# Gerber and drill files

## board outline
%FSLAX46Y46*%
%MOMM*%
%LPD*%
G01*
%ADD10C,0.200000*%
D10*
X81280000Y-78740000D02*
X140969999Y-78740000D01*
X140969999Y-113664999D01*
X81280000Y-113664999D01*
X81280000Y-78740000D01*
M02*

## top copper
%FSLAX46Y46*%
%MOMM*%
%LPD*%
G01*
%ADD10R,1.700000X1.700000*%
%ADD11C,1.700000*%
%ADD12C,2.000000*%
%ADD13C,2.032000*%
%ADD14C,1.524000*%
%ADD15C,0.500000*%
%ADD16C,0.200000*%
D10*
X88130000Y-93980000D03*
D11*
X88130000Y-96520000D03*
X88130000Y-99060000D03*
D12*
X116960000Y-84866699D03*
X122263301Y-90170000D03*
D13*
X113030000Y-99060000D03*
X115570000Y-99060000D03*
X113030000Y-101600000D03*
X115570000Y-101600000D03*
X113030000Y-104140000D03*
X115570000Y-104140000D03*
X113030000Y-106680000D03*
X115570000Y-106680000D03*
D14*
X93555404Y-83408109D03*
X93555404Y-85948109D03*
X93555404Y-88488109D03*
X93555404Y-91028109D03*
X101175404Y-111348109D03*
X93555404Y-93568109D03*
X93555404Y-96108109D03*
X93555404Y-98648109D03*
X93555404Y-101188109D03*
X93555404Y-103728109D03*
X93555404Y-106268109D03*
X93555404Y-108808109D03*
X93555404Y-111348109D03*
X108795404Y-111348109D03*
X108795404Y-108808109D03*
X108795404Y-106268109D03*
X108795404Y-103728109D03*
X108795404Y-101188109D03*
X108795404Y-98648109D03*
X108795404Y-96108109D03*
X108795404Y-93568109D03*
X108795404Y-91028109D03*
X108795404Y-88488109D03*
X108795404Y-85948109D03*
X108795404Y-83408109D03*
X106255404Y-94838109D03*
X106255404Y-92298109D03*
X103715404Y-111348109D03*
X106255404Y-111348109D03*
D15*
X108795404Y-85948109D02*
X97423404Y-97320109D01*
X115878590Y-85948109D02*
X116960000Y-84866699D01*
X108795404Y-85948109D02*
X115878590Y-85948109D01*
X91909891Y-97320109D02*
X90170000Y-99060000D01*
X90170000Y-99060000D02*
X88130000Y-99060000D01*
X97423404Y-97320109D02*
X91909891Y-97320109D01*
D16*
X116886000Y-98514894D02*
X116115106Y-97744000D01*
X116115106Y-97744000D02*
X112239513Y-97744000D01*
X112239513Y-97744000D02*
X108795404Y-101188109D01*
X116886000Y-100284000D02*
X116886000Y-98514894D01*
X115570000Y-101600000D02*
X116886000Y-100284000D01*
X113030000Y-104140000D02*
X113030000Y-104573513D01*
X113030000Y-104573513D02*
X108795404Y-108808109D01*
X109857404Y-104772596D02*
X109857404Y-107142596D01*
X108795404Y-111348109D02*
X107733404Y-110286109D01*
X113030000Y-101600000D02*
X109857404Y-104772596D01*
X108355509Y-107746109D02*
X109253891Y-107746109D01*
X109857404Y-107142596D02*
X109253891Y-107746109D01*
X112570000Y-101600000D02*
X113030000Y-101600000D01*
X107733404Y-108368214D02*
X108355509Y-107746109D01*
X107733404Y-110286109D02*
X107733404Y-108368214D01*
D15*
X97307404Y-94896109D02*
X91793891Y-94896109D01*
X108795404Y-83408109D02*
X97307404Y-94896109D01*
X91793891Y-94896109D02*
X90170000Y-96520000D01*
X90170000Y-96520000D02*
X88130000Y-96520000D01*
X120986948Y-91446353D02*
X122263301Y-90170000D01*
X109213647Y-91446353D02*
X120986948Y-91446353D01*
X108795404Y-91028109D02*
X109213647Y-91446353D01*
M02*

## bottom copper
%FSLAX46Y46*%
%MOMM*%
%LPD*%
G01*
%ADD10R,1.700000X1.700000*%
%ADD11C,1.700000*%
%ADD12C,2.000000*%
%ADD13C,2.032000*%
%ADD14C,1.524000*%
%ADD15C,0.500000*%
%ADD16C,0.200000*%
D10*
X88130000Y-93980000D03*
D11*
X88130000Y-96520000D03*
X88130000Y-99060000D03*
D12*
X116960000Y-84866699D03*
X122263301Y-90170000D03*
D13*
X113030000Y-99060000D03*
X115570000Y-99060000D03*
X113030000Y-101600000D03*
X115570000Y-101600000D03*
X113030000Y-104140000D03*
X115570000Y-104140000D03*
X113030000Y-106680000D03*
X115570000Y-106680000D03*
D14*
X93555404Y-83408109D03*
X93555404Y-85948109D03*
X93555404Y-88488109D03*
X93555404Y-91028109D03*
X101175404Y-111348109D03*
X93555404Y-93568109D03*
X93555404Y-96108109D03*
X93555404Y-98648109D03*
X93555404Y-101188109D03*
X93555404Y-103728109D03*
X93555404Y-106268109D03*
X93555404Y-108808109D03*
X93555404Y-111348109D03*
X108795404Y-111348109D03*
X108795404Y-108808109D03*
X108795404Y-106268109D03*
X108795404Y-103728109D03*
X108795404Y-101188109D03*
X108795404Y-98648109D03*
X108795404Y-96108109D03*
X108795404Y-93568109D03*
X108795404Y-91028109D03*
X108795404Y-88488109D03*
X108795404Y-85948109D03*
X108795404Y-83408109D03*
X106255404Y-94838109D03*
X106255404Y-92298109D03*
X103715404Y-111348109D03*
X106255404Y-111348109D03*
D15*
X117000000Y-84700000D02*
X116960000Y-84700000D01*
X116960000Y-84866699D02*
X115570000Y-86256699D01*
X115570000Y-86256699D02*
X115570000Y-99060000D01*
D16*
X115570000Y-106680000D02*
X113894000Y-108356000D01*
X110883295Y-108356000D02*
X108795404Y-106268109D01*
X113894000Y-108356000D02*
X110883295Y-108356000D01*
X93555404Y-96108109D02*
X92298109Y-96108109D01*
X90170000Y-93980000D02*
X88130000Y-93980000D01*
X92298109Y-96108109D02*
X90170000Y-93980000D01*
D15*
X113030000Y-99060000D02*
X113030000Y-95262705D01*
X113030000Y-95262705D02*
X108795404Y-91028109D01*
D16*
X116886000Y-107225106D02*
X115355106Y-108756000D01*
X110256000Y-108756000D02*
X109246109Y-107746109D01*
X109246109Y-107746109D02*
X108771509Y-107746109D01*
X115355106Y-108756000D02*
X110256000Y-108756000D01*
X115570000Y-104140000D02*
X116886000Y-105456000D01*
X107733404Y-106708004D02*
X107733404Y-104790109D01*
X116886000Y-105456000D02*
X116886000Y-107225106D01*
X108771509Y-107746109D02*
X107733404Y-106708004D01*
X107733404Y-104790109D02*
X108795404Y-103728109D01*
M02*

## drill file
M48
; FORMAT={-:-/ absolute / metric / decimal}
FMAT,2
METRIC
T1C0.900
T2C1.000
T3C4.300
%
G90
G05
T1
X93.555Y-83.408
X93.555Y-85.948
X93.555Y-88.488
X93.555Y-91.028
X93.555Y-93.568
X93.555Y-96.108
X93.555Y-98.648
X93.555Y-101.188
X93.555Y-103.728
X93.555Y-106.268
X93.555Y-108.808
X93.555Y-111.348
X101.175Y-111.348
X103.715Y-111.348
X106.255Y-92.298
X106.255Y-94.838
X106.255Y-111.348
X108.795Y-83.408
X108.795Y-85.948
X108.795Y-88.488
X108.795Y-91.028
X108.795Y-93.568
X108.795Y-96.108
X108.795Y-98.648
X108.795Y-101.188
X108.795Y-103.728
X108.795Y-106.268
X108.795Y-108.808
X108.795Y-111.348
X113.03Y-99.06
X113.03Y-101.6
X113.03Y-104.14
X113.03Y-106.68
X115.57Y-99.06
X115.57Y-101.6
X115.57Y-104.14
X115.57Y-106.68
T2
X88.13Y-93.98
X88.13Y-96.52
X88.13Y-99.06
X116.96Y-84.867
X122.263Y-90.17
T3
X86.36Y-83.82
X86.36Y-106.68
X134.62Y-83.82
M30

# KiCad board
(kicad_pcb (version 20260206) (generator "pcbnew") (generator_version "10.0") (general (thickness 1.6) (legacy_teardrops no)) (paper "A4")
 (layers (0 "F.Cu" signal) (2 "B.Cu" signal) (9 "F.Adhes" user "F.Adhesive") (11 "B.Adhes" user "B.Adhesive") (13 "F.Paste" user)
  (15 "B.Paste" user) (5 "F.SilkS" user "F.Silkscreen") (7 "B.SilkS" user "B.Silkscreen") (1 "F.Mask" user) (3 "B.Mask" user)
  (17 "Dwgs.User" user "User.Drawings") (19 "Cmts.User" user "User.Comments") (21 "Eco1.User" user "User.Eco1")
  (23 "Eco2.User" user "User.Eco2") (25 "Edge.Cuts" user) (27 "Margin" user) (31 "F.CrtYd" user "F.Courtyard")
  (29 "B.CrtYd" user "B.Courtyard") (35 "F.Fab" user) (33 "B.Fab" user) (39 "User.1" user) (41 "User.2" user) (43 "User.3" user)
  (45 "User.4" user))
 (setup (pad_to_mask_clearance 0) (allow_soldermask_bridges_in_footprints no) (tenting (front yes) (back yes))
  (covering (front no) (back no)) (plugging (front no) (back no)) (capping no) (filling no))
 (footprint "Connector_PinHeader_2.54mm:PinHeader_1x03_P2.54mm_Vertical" (layer "F.Cu") (at 88.13 93.98)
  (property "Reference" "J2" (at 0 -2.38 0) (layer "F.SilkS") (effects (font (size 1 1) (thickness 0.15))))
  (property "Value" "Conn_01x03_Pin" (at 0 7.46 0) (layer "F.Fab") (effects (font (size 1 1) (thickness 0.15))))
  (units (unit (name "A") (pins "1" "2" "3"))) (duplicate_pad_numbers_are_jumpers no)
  (pad "1" thru_hole rect (at 0 0) (size 1.7 1.7) (drill 1) (layers "*.Cu" "*.Mask") (remove_unused_layers no) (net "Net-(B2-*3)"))
  (pad "2" thru_hole circle (at 0 2.54) (size 1.7 1.7) (drill 1) (layers "*.Cu" "*.Mask") (remove_unused_layers no) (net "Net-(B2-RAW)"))
  (pad "3" thru_hole circle (at 0 5.08) (size 1.7 1.7) (drill 1) (layers "*.Cu" "*.Mask") (remove_unused_layers no) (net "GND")))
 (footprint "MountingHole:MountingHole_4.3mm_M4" (layer "F.Cu") (at 86.36 83.82)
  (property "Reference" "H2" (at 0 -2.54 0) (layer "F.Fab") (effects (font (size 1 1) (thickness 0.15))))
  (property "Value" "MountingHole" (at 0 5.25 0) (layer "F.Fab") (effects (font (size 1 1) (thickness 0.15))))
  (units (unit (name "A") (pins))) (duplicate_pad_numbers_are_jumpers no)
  (pad "" np_thru_hole circle (at 0 0) (size 4.3 4.3) (drill 4.3) (layers "*.Cu" "*.Mask")))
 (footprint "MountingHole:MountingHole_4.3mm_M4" (layer "F.Cu") (at 134.62 83.82)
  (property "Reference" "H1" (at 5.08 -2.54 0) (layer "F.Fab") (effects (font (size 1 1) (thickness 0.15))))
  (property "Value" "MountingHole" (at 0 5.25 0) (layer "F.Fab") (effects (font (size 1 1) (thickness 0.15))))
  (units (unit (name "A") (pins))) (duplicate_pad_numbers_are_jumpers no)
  (pad "" np_thru_hole circle (at 0 0) (size 4.3 4.3) (drill 4.3) (layers "*.Cu" "*.Mask")))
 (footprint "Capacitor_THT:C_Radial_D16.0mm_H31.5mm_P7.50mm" (layer "F.Cu") (at 116.96 84.866699 -45)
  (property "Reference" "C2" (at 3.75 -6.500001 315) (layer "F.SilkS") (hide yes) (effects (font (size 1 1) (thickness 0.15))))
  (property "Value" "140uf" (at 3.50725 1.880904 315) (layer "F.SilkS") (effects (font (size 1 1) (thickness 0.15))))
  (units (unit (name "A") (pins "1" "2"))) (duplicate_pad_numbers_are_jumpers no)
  (pad "1" thru_hole circle (at 0 0) (size 2 2) (drill 1) (layers "*.Cu" "*.Mask") (remove_unused_layers no) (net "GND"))
  (pad "2" thru_hole circle (at 7.5 0 315) (size 2 2) (drill 1) (layers "*.Cu" "*.Mask") (remove_unused_layers no) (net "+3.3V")))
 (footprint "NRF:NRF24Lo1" (layer "F.Cu") (at 125.73 104.775)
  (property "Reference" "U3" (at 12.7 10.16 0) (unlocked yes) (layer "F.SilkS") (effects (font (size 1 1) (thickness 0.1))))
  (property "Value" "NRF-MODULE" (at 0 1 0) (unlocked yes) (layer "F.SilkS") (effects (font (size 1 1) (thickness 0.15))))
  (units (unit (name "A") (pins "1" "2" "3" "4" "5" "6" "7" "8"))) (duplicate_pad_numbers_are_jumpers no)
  (pad "1" thru_hole circle (at -12.7 -5.715) (size 2.032 2.032) (drill 0.9) (layers "*.Cu" "*.Mask") (remove_unused_layers no)
   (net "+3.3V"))
  (pad "2" thru_hole circle (at -10.16 -5.715) (size 2.032 2.032) (drill 0.9) (layers "*.Cu" "*.Mask") (remove_unused_layers no) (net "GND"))
  (pad "3" thru_hole circle (at -12.7 -3.175) (size 2.032 2.032) (drill 0.9) (layers "*.Cu" "*.Mask") (remove_unused_layers no) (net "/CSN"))
  (pad "4" thru_hole circle (at -10.16 -3.175) (size 2.032 2.032) (drill 0.9) (layers "*.Cu" "*.Mask") (remove_unused_layers no) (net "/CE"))
  (pad "5" thru_hole circle (at -12.7 -0.635) (size 2.032 2.032) (drill 0.9) (layers "*.Cu" "*.Mask") (remove_unused_layers no)
   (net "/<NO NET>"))
  (pad "6" thru_hole circle (at -10.16 -0.635) (size 2.032 2.032) (drill 0.9) (layers "*.Cu" "*.Mask") (remove_unused_layers no)
   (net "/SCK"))
  (pad "7" thru_hole circle (at -12.7 1.905) (size 2.032 2.032) (drill 0.9) (layers "*.Cu" "*.Mask") (remove_unused_layers no)
   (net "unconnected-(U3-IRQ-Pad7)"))
  (pad "8" thru_hole circle (at -10.16 1.905) (size 2.032 2.032) (drill 0.9) (layers "*.Cu" "*.Mask") (remove_unused_layers no)
   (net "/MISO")))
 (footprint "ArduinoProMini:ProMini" (layer "F.Cu") (at 101.175404 96.108109)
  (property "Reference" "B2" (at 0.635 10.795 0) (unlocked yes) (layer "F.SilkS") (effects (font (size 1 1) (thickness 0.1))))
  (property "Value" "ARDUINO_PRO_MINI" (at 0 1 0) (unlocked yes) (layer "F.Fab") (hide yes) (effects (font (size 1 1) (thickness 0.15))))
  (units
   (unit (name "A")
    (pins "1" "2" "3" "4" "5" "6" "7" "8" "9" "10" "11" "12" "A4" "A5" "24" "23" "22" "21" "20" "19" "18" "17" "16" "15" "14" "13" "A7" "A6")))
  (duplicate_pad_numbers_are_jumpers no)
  (pad "1" thru_hole circle (at -7.62 -12.7) (size 1.524 1.524) (drill 0.9) (layers "*.Cu" "*.Mask") (remove_unused_layers no)
   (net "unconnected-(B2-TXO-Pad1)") (thermal_bridge_angle 90))
  (pad "2" thru_hole circle (at -7.62 -10.16) (size 1.524 1.524) (drill 0.9) (layers "*.Cu" "*.Mask") (remove_unused_layers no)
   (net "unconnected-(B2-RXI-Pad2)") (thermal_bridge_angle 90))
  (pad "3" thru_hole circle (at -7.62 -7.62) (size 1.524 1.524) (drill 0.9) (layers "*.Cu" "*.Mask") (remove_unused_layers no)
   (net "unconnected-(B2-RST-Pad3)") (thermal_bridge_angle 90))
  (pad "4" thru_hole circle (at -7.62 -5.08) (size 1.524 1.524) (drill 0.9) (layers "*.Cu" "*.Mask") (remove_unused_layers no)
   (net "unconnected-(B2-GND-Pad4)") (thermal_bridge_angle 90))
  (pad "4" thru_hole circle (at 0 15.24) (size 1.524 1.524) (drill 0.9) (layers "*.Cu" "*.Mask") (remove_unused_layers no)
   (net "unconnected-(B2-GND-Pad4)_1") (thermal_bridge_angle 90))
  (pad "5" thru_hole circle (at -7.62 -2.54) (size 1.524 1.524) (drill 0.9) (layers "*.Cu" "*.Mask") (remove_unused_layers no)
   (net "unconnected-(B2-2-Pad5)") (thermal_bridge_angle 90))
  (pad "6" thru_hole circle (at -7.62 0) (size 1.524 1.524) (drill 0.9) (layers "*.Cu" "*.Mask") (remove_unused_layers no)
   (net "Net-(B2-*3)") (thermal_bridge_angle 90))
  (pad "7" thru_hole circle (at -7.62 2.54) (size 1.524 1.524) (drill 0.9) (layers "*.Cu" "*.Mask") (remove_unused_layers no)
   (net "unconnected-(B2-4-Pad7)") (thermal_bridge_angle 90))
  (pad "8" thru_hole circle (at -7.62 5.08) (size 1.524 1.524) (drill 0.9) (layers "*.Cu" "*.Mask") (remove_unused_layers no)
   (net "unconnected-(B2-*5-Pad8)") (thermal_bridge_angle 90))
  (pad "9" thru_hole circle (at -7.62 7.62) (size 1.524 1.524) (drill 0.9) (layers "*.Cu" "*.Mask") (remove_unused_layers no)
   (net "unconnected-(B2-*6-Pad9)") (thermal_bridge_angle 90))
  (pad "10" thru_hole circle (at -7.62 10.16) (size 1.524 1.524) (drill 0.9) (layers "*.Cu" "*.Mask") (remove_unused_layers no)
   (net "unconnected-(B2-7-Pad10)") (thermal_bridge_angle 90))
  (pad "11" thru_hole circle (at -7.62 12.7) (size 1.524 1.524) (drill 0.9) (layers "*.Cu" "*.Mask") (remove_unused_layers no)
   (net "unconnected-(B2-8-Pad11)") (thermal_bridge_angle 90))
  (pad "12" thru_hole circle (at -7.62 15.24) (size 1.524 1.524) (drill 0.9) (layers "*.Cu" "*.Mask") (remove_unused_layers no)
   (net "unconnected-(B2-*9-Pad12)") (thermal_bridge_angle 90))
  (pad "13" thru_hole circle (at 7.62 15.24) (size 1.524 1.524) (drill 0.9) (layers "*.Cu" "*.Mask") (remove_unused_layers no) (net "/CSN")
   (thermal_bridge_angle 90))
  (pad "14" thru_hole circle (at 7.62 12.7) (size 1.524 1.524) (drill 0.9) (layers "*.Cu" "*.Mask") (remove_unused_layers no)
   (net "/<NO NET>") (thermal_bridge_angle 90))
  (pad "15" thru_hole circle (at 7.62 10.16) (size 1.524 1.524) (drill 0.9) (layers "*.Cu" "*.Mask") (remove_unused_layers no) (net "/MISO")
   (thermal_bridge_angle 90))
  (pad "16" thru_hole circle (at 7.62 7.62) (size 1.524 1.524) (drill 0.9) (layers "*.Cu" "*.Mask") (remove_unused_layers no) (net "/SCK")
   (thermal_bridge_angle 90))
  (pad "17" thru_hole circle (at 7.62 5.08) (size 1.524 1.524) (drill 0.9) (layers "*.Cu" "*.Mask") (remove_unused_layers no) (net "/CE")
   (thermal_bridge_angle 90))
  (pad "18" thru_hole circle (at 7.62 2.54) (size 1.524 1.524) (drill 0.9) (layers "*.Cu" "*.Mask") (remove_unused_layers no)
   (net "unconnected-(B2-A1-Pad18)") (thermal_bridge_angle 90))
  (pad "19" thru_hole circle (at 7.62 0) (size 1.524 1.524) (drill 0.9) (layers "*.Cu" "*.Mask") (remove_unused_layers no)
   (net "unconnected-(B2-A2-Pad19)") (thermal_bridge_angle 90))
  (pad "20" thru_hole circle (at 7.62 -2.54) (size 1.524 1.524) (drill 0.9) (layers "*.Cu" "*.Mask") (remove_unused_layers no)
   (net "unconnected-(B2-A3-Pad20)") (thermal_bridge_angle 90))
  (pad "21" thru_hole circle (at 7.62 -5.08) (size 1.524 1.524) (drill 0.9) (layers "*.Cu" "*.Mask") (remove_unused_layers no) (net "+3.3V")
   (thermal_bridge_angle 90))
  (pad "22" thru_hole circle (at 7.62 -7.62) (size 1.524 1.524) (drill 0.9) (layers "*.Cu" "*.Mask") (remove_unused_layers no)
   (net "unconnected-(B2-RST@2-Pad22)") (thermal_bridge_angle 90))
  (pad "23" thru_hole circle (at 7.62 -10.16) (size 1.524 1.524) (drill 0.9) (layers "*.Cu" "*.Mask") (remove_unused_layers no) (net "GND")
   (thermal_bridge_angle 90))
  (pad "24" thru_hole circle (at 7.62 -12.7) (size 1.524 1.524) (drill 0.9) (layers "*.Cu" "*.Mask") (remove_unused_layers no)
   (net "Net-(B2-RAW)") (thermal_bridge_angle 90))
  (pad "A4" thru_hole circle (at 5.08 -1.27) (size 1.524 1.524) (drill 0.9) (layers "*.Cu" "*.Mask") (remove_unused_layers no)
   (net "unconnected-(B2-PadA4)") (thermal_bridge_angle 90))
  (pad "A5" thru_hole circle (at 5.08 -3.81) (size 1.524 1.524) (drill 0.9) (layers "*.Cu" "*.Mask") (remove_unused_layers no)
   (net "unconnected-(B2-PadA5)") (thermal_bridge_angle 90))
  (pad "A6" thru_hole circle (at 2.54 15.24) (size 1.524 1.524) (drill 0.9) (layers "*.Cu" "*.Mask") (remove_unused_layers no)
   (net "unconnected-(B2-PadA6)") (thermal_bridge_angle 90))
  (pad "A7" thru_hole circle (at 5.08 15.24) (size 1.524 1.524) (drill 0.9) (layers "*.Cu" "*.Mask") (remove_unused_layers no)
   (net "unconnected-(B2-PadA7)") (thermal_bridge_angle 90)))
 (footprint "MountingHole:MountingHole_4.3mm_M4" (layer "F.Cu") (at 86.36 106.68)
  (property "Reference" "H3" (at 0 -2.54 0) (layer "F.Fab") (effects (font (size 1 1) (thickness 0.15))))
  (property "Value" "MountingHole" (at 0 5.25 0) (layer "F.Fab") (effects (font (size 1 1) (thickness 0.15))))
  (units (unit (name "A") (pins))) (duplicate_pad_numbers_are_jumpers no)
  (pad "" np_thru_hole circle (at 0 0) (size 4.3 4.3) (drill 4.3) (layers "*.Cu" "*.Mask")))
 (gr_rect (start 81.28 78.74) (end 140.969999 113.664999) (stroke (width 0.2) (type default)) (fill no) (layer "Edge.Cuts"))
 (segment (start 108.795404 85.948109) (end 97.423404 97.320109) (width 0.5) (layer "F.Cu") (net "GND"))
 (segment (start 115.87859 85.948109) (end 116.96 84.866699) (width 0.5) (layer "F.Cu") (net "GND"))
 (segment (start 108.795404 85.948109) (end 115.87859 85.948109) (width 0.5) (layer "F.Cu") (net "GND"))
 (segment (start 91.909891 97.320109) (end 90.17 99.06) (width 0.5) (layer "F.Cu") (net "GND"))
 (segment (start 90.17 99.06) (end 88.13 99.06) (width 0.5) (layer "F.Cu") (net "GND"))
 (segment (start 97.423404 97.320109) (end 91.909891 97.320109) (width 0.5) (layer "F.Cu") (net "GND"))
 (segment (start 117 84.7) (end 116.96 84.7) (width 0.5) (layer "B.Cu") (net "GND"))
 (segment (start 116.96 84.866699) (end 115.57 86.256699) (width 0.5) (layer "B.Cu") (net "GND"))
 (segment (start 115.57 86.256699) (end 115.57 99.06) (width 0.5) (layer "B.Cu") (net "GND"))
 (segment (start 116.886 98.514894) (end 116.115106 97.744) (width 0.2) (layer "F.Cu") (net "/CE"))
 (segment (start 116.115106 97.744) (end 112.239513 97.744) (width 0.2) (layer "F.Cu") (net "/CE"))
 (segment (start 112.239513 97.744) (end 108.795404 101.188109) (width 0.2) (layer "F.Cu") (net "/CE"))
 (segment (start 116.886 100.284) (end 116.886 98.514894) (width 0.2) (layer "F.Cu") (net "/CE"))
 (segment (start 115.57 101.6) (end 116.886 100.284) (width 0.2) (layer "F.Cu") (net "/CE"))
 (segment (start 115.57 106.68) (end 113.894 108.356) (width 0.2) (layer "B.Cu") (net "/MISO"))
 (segment (start 110.883295 108.356) (end 108.795404 106.268109) (width 0.2) (layer "B.Cu") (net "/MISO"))
 (segment (start 113.894 108.356) (end 110.883295 108.356) (width 0.2) (layer "B.Cu") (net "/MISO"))
 (segment (start 113.03 104.14) (end 113.03 104.573513) (width 0.2) (layer "F.Cu") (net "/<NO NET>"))
 (segment (start 113.03 104.573513) (end 108.795404 108.808109) (width 0.2) (layer "F.Cu") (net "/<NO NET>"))
 (segment (start 109.857404 104.772596) (end 109.857404 107.142596) (width 0.2) (layer "F.Cu") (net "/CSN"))
 (segment (start 108.795404 111.348109) (end 107.733404 110.286109) (width 0.2) (layer "F.Cu") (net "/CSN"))
 (segment (start 113.03 101.6) (end 109.857404 104.772596) (width 0.2) (layer "F.Cu") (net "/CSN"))
 (segment (start 108.355509 107.746109) (end 109.253891 107.746109) (width 0.2) (layer "F.Cu") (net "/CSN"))
 (segment (start 109.857404 107.142596) (end 109.253891 107.746109) (width 0.2) (layer "F.Cu") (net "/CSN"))
 (segment (start 112.57 101.6) (end 113.03 101.6) (width 0.2) (layer "F.Cu") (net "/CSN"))
 (segment (start 107.733404 108.368214) (end 108.355509 107.746109) (width 0.2) (layer "F.Cu") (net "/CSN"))
 (segment (start 107.733404 110.286109) (end 107.733404 108.368214) (width 0.2) (layer "F.Cu") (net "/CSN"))
 (segment (start 93.555404 96.108109) (end 92.298109 96.108109) (width 0.2) (layer "B.Cu") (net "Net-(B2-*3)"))
 (segment (start 90.17 93.98) (end 88.13 93.98) (width 0.2) (layer "B.Cu") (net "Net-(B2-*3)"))
 (segment (start 92.298109 96.108109) (end 90.17 93.98) (width 0.2) (layer "B.Cu") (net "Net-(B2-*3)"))
 (segment (start 97.307404 94.896109) (end 91.793891 94.896109) (width 0.5) (layer "F.Cu") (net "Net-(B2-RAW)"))
 (segment (start 108.795404 83.408109) (end 97.307404 94.896109) (width 0.5) (layer "F.Cu") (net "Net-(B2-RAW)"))
 (segment (start 91.793891 94.896109) (end 90.17 96.52) (width 0.5) (layer "F.Cu") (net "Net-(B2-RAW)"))
 (segment (start 90.17 96.52) (end 88.13 96.52) (width 0.5) (layer "F.Cu") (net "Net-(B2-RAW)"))
 (segment (start 120.986948 91.446353) (end 122.263301 90.17) (width 0.5) (layer "F.Cu") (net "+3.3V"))
 (segment (start 109.213647 91.446353) (end 120.986948 91.446353) (width 0.5) (layer "F.Cu") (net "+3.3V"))
 (segment (start 108.795404 91.028109) (end 109.213647 91.446353) (width 0.5) (layer "F.Cu") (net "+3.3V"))
 (segment (start 113.03 99.06) (end 113.03 95.262705) (width 0.5) (layer "B.Cu") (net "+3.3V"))
 (segment (start 113.03 95.262705) (end 108.795404 91.028109) (width 0.5) (layer "B.Cu") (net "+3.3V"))
 (segment (start 116.886 107.225106) (end 115.355106 108.756) (width 0.2) (layer "B.Cu") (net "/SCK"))
 (segment (start 110.256 108.756) (end 109.246109 107.746109) (width 0.2) (layer "B.Cu") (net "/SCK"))
 (segment (start 109.246109 107.746109) (end 108.771509 107.746109) (width 0.2) (layer "B.Cu") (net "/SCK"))
 (segment (start 115.355106 108.756) (end 110.256 108.756) (width 0.2) (layer "B.Cu") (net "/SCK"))
 (segment (start 115.57 104.14) (end 116.886 105.456) (width 0.2) (layer "B.Cu") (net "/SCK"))
 (segment (start 107.733404 106.708004) (end 107.733404 104.790109) (width 0.2) (layer "B.Cu") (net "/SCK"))
 (segment (start 116.886 105.456) (end 116.886 107.225106) (width 0.2) (layer "B.Cu") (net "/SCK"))
 (segment (start 108.771509 107.746109) (end 107.733404 106.708004) (width 0.2) (layer "B.Cu") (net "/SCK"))
 (segment (start 107.733404 104.790109) (end 108.795404 103.728109) (width 0.2) (layer "B.Cu") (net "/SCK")))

